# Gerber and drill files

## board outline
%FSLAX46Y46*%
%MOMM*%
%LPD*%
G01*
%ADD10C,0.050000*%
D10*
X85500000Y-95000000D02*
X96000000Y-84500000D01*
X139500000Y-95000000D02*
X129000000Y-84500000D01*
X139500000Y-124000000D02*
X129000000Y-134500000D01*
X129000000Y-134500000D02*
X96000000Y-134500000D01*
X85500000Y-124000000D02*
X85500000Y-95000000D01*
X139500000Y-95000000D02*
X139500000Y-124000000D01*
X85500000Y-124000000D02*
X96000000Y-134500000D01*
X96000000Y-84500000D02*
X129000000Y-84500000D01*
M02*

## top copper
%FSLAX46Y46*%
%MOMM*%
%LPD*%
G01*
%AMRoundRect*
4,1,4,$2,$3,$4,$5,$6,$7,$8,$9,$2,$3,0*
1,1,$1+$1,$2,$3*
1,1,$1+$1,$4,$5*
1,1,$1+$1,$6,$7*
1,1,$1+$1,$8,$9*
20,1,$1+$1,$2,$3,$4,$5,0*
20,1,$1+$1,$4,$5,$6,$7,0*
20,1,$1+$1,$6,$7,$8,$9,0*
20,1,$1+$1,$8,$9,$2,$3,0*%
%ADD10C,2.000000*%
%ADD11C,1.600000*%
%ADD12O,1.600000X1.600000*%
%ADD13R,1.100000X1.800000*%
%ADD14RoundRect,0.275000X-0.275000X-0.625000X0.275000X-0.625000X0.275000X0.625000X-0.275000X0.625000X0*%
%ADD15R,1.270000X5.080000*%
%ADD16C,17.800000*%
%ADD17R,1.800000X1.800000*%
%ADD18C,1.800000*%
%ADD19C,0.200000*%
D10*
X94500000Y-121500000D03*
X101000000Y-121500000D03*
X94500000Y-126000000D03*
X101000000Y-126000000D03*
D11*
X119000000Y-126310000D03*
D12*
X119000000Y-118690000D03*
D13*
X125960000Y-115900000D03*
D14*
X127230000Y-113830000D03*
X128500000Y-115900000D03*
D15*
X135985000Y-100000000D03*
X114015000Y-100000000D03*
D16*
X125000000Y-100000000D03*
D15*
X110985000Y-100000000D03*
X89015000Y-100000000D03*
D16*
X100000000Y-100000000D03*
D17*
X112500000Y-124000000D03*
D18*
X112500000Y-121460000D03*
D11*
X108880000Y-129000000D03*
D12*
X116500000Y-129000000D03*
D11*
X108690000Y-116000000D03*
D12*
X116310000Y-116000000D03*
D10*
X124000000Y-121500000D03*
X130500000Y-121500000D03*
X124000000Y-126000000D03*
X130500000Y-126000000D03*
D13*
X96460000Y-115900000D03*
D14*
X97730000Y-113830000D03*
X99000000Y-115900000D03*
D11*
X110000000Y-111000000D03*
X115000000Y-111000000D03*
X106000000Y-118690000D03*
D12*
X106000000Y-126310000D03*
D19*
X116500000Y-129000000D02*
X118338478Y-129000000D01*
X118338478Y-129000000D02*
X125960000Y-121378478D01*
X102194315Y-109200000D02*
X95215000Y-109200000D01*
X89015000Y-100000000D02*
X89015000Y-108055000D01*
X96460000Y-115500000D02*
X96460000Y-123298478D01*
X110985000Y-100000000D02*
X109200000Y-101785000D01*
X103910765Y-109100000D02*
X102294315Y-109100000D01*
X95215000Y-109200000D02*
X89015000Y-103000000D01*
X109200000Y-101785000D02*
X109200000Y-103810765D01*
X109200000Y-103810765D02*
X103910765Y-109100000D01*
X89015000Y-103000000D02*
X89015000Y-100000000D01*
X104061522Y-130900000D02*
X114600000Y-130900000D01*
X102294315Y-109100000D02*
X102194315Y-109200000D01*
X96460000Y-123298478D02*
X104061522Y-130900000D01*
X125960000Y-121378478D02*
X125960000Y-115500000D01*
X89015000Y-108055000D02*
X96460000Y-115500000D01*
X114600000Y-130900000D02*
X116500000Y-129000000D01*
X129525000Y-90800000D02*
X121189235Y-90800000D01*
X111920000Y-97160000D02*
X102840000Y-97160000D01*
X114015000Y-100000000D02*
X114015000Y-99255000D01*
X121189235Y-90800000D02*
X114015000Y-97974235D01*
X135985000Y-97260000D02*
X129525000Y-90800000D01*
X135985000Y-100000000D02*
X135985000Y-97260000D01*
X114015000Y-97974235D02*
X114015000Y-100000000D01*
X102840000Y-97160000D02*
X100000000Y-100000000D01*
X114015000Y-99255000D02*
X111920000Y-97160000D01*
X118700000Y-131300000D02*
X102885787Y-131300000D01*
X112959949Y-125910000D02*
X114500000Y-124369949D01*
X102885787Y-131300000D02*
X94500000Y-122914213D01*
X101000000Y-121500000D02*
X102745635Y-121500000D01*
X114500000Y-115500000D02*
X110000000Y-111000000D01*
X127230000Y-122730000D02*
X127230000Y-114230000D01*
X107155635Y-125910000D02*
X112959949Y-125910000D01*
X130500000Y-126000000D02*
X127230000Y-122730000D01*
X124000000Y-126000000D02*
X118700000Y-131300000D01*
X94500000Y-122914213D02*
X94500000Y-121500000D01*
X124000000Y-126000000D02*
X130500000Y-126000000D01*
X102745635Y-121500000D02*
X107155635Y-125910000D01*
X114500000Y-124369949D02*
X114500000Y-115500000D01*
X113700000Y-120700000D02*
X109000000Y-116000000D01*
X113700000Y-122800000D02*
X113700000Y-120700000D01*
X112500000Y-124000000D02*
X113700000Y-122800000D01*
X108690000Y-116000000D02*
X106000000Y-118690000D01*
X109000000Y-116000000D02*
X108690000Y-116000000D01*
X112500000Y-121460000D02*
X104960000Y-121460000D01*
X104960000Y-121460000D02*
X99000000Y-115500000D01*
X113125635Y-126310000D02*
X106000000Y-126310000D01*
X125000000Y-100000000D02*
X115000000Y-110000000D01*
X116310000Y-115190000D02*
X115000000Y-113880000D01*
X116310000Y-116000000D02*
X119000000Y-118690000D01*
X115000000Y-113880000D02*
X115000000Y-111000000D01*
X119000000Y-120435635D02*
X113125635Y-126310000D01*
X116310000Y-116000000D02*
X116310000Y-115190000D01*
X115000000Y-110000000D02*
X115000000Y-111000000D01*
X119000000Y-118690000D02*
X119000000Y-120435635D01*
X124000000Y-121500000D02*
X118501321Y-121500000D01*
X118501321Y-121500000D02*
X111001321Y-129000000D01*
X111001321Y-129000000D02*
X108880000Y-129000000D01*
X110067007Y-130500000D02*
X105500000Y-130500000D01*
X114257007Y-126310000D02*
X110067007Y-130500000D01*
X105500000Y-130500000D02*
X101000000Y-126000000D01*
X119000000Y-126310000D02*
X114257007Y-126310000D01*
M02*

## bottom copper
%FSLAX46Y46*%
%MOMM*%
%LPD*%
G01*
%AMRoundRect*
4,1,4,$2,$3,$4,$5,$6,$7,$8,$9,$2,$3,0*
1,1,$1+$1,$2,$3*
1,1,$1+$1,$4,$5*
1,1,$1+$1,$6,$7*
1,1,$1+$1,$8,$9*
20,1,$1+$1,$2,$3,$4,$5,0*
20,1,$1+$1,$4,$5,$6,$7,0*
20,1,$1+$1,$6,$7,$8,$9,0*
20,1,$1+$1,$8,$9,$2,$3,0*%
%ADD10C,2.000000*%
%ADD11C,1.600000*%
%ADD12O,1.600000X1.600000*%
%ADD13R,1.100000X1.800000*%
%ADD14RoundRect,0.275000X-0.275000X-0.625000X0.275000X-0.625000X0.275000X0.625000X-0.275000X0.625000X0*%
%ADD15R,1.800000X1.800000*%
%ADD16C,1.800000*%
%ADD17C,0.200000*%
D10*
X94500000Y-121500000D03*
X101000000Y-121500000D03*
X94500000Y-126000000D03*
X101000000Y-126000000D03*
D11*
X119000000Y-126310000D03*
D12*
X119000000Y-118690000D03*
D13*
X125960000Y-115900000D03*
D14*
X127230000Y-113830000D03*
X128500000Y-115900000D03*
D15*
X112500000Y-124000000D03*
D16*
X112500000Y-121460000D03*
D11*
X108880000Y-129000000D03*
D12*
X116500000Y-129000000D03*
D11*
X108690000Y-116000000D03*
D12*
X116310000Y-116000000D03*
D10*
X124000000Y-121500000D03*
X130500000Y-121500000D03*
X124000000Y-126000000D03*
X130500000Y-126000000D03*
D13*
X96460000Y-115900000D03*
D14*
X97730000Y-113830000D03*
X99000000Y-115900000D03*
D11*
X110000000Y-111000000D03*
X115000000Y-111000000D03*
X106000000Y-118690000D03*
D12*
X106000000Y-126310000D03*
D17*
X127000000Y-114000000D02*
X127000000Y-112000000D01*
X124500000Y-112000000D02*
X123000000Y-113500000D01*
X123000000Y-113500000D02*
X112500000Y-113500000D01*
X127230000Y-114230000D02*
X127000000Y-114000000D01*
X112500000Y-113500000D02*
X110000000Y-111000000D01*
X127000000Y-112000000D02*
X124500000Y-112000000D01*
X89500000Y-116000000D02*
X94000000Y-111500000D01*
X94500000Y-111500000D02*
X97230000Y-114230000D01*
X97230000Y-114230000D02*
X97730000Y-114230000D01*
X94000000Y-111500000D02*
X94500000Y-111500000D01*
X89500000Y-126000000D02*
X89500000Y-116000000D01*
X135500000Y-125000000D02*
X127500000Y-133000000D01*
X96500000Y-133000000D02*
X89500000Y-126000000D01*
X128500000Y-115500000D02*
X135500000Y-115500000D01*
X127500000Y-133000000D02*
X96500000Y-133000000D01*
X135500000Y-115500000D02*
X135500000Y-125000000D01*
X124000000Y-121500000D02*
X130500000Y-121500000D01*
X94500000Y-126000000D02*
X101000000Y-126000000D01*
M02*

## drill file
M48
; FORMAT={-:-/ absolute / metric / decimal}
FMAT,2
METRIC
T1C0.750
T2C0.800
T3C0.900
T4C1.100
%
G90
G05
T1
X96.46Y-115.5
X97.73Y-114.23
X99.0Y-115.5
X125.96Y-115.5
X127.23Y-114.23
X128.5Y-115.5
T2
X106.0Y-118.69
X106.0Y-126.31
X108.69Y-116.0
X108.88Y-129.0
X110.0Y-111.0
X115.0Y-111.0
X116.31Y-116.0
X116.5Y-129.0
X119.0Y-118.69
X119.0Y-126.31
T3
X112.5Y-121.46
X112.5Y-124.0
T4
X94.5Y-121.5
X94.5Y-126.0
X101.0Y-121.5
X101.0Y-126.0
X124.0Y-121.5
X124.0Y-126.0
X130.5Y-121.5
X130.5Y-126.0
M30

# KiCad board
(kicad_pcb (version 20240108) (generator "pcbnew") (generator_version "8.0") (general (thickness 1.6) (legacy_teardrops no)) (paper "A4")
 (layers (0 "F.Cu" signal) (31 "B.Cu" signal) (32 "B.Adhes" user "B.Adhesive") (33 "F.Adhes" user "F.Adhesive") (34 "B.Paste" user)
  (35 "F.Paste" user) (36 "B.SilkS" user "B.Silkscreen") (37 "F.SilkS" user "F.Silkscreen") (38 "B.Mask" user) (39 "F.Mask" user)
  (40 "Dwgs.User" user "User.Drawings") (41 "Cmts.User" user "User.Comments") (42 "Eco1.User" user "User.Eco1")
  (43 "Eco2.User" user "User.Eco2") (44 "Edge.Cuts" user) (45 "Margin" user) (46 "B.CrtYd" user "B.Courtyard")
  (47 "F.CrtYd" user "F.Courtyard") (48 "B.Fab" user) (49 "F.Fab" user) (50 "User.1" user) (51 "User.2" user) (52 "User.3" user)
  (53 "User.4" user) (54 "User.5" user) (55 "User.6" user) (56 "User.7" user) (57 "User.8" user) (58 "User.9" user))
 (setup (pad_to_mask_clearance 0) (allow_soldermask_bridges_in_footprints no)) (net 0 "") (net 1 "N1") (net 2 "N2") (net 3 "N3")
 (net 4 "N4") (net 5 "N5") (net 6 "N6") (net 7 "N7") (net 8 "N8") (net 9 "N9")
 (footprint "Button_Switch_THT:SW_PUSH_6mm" (layer "F.Cu") (at 94.5 121.5)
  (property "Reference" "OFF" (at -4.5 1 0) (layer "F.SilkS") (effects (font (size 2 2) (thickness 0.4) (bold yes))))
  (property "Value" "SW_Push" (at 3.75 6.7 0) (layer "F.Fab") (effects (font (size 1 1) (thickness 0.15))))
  (pad "1" thru_hole circle (at 0 0 90) (size 2 2) (drill 1.1) (layers "*.Cu" "*.Mask") (remove_unused_layers no) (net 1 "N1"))
  (pad "1" thru_hole circle (at 6.5 0 90) (size 2 2) (drill 1.1) (layers "*.Cu" "*.Mask") (remove_unused_layers no) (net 1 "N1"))
  (pad "2" thru_hole circle (at 0 4.5 90) (size 2 2) (drill 1.1) (layers "*.Cu" "*.Mask") (remove_unused_layers no) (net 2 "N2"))
  (pad "2" thru_hole circle (at 6.5 4.5 90) (size 2 2) (drill 1.1) (layers "*.Cu" "*.Mask") (remove_unused_layers no) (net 2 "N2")))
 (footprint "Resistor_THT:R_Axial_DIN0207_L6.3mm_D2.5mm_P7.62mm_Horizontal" (layer "F.Cu") (at 119 126.31 90)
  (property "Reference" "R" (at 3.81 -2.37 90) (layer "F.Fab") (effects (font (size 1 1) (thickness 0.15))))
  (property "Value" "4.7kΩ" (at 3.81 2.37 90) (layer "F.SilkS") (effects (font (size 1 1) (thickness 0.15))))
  (pad "1" thru_hole circle (at 0 0 90) (size 1.6 1.6) (drill 0.8) (layers "*.Cu" "*.Mask") (remove_unused_layers no) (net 2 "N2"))
  (pad "2" thru_hole oval (at 7.62 0 90) (size 1.6 1.6) (drill 0.8) (layers "*.Cu" "*.Mask") (remove_unused_layers no) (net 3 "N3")))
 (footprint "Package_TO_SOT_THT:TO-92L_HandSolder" (layer "F.Cu") (at 125.96 115.5)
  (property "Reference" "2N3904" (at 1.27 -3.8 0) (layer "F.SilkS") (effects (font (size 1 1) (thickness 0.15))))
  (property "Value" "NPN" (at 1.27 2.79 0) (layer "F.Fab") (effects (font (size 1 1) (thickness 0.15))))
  (pad "1" thru_hole rect (at 0 0) (size 1.1 1.8) (drill 0.75 (offset 0 0.4)) (layers "*.Cu" "*.Mask") (remove_unused_layers no)
   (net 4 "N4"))
  (pad "2" thru_hole roundrect (at 1.27 -1.27) (size 1.1 1.8) (drill 0.75 (offset 0 -0.4)) (layers "*.Cu" "*.Mask")
   (remove_unused_layers no) (roundrect_rratio 0.25) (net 1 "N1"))
  (pad "3" thru_hole roundrect (at 2.54 0) (size 1.1 1.8) (drill 0.75 (offset 0 0.4)) (layers "*.Cu" "*.Mask") (remove_unused_layers no)
   (roundrect_rratio 0.25) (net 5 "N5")))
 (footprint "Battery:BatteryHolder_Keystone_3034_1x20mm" (layer "F.Cu") (at 125 100 180)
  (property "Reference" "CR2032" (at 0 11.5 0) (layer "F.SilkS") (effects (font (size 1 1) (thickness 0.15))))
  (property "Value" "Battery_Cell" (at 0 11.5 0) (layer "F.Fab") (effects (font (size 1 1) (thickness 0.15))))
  (pad "1" smd rect (at -10.985 0 180) (size 1.27 5.08) (layers "F.Cu" "F.Paste" "F.Mask") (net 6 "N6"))
  (pad "1" smd rect (at 10.985 0 180) (size 1.27 5.08) (layers "F.Cu" "F.Paste" "F.Mask") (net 6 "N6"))
  (pad "2" smd circle (at 0 0 180) (size 17.8 17.8) (layers "F.Cu" "F.Mask") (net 3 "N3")))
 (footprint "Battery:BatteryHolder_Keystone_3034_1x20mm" (layer "F.Cu") (at 100 100 180)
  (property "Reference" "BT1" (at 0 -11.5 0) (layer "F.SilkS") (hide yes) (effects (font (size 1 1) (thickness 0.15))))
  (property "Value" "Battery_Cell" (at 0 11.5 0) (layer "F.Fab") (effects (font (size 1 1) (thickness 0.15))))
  (pad "1" smd rect (at -10.985 0 180) (size 1.27 5.08) (layers "F.Cu" "F.Paste" "F.Mask") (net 4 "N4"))
  (pad "1" smd rect (at 10.985 0 180) (size 1.27 5.08) (layers "F.Cu" "F.Paste" "F.Mask") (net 4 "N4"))
  (pad "2" smd circle (at 0 0 180) (size 17.8 17.8) (layers "F.Cu" "F.Mask") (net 6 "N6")))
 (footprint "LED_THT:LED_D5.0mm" (layer "F.Cu") (at 112.5 124 90)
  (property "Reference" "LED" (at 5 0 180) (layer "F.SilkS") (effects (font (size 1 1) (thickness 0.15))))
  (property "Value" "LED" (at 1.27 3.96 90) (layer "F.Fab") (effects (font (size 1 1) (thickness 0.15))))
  (pad "1" thru_hole rect (at 0 0 90) (size 1.8 1.8) (drill 0.9) (layers "*.Cu" "*.Mask") (remove_unused_layers no) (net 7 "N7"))
  (pad "2" thru_hole circle (at 2.54 0 90) (size 1.8 1.8) (drill 0.9) (layers "*.Cu" "*.Mask") (remove_unused_layers no) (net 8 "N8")))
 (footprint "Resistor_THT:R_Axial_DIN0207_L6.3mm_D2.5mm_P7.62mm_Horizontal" (layer "F.Cu") (at 108.88 129)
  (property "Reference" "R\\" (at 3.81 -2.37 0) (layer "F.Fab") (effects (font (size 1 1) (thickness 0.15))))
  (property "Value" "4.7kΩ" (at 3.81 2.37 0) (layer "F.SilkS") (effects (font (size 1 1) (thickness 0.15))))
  (pad "1" thru_hole circle (at 0 0) (size 1.6 1.6) (drill 0.8) (layers "*.Cu" "*.Mask") (remove_unused_layers no) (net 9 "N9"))
  (pad "2" thru_hole oval (at 7.62 0) (size 1.6 1.6) (drill 0.8) (layers "*.Cu" "*.Mask") (remove_unused_layers no) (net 4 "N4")))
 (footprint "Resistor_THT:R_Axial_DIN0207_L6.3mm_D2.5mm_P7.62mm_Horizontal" (layer "F.Cu") (at 108.69 116)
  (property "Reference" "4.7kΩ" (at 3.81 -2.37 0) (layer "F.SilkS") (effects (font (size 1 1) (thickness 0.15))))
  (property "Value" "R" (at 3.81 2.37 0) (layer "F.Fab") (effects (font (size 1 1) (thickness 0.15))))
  (pad "1" thru_hole circle (at 0 0) (size 1.6 1.6) (drill 0.8) (layers "*.Cu" "*.Mask") (remove_unused_layers no) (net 7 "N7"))
  (pad "2" thru_hole oval (at 7.62 0) (size 1.6 1.6) (drill 0.8) (layers "*.Cu" "*.Mask") (remove_unused_layers no) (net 3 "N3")))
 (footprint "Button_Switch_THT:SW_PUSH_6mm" (layer "F.Cu") (at 124 121.5)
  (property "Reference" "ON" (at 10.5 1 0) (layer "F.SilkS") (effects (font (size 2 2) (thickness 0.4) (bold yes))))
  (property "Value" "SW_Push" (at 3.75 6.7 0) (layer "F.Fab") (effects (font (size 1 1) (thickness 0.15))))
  (pad "1" thru_hole circle (at 0 0 90) (size 2 2) (drill 1.1) (layers "*.Cu" "*.Mask") (remove_unused_layers no) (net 9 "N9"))
  (pad "1" thru_hole circle (at 6.5 0 90) (size 2 2) (drill 1.1) (layers "*.Cu" "*.Mask") (remove_unused_layers no) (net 9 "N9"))
  (pad "2" thru_hole circle (at 0 4.5 90) (size 2 2) (drill 1.1) (layers "*.Cu" "*.Mask") (remove_unused_layers no) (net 1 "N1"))
  (pad "2" thru_hole circle (at 6.5 4.5 90) (size 2 2) (drill 1.1) (layers "*.Cu" "*.Mask") (remove_unused_layers no) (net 1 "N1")))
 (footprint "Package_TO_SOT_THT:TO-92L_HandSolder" (layer "F.Cu") (at 96.46 115.5)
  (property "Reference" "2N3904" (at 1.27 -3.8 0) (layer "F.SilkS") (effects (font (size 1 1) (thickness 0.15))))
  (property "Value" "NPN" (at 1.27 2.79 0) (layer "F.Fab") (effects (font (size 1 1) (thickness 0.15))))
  (pad "1" thru_hole rect (at 0 0) (size 1.1 1.8) (drill 0.75 (offset 0 0.4)) (layers "*.Cu" "*.Mask") (remove_unused_layers no)
   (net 4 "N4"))
  (pad "2" thru_hole roundrect (at 1.27 -1.27) (size 1.1 1.8) (drill 0.75 (offset 0 -0.4)) (layers "*.Cu" "*.Mask")
   (remove_unused_layers no) (roundrect_rratio 0.25) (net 5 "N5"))
  (pad "3" thru_hole roundrect (at 2.54 0) (size 1.1 1.8) (drill 0.75 (offset 0 0.4)) (layers "*.Cu" "*.Mask") (remove_unused_layers no)
   (roundrect_rratio 0.25) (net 8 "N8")))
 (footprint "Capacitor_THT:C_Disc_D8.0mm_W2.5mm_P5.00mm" (layer "F.Cu") (at 110 111)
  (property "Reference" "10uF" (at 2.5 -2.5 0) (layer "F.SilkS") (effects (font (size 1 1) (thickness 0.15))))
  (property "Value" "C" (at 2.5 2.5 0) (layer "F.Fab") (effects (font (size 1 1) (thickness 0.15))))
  (pad "1" thru_hole circle (at 0 0) (size 1.6 1.6) (drill 0.8) (layers "*.Cu" "*.Mask") (remove_unused_layers no) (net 1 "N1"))
  (pad "2" thru_hole circle (at 5 0) (size 1.6 1.6) (drill 0.8) (layers "*.Cu" "*.Mask") (remove_unused_layers no) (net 3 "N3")))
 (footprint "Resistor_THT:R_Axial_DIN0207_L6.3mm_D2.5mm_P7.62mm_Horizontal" (layer "F.Cu") (at 106 118.69 -90)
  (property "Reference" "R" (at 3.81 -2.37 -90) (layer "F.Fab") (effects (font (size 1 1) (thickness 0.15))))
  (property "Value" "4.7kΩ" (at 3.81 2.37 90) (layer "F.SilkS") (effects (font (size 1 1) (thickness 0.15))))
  (pad "1" thru_hole circle (at 0 0 270) (size 1.6 1.6) (drill 0.8) (layers "*.Cu" "*.Mask") (remove_unused_layers no) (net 7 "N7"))
  (pad "2" thru_hole oval (at 7.62 0 270) (size 1.6 1.6) (drill 0.8) (layers "*.Cu" "*.Mask") (remove_unused_layers no) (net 3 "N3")))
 (gr_line (start 85.5 95) (end 96 84.5) (stroke (width 0.05) (type default)) (layer "Edge.Cuts"))
 (gr_line (start 139.5 95) (end 129 84.5) (stroke (width 0.05) (type default)) (layer "Edge.Cuts"))
 (gr_line (start 139.5 124) (end 129 134.5) (stroke (width 0.05) (type default)) (layer "Edge.Cuts"))
 (gr_line (start 129 134.5) (end 96 134.5) (stroke (width 0.05) (type default)) (layer "Edge.Cuts"))
 (gr_line (start 85.5 124) (end 85.5 95) (stroke (width 0.05) (type default)) (layer "Edge.Cuts"))
 (gr_line (start 139.5 95) (end 139.5 124) (stroke (width 0.05) (type default)) (layer "Edge.Cuts"))
 (gr_line (start 85.5 124) (end 96 134.5) (stroke (width 0.05) (type default)) (layer "Edge.Cuts"))
 (gr_line (start 96 84.5) (end 129 84.5) (stroke (width 0.05) (type default)) (layer "Edge.Cuts"))
 (segment (start 116.5 129) (end 118.338478 129) (width 0.2) (layer "F.Cu") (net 4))
 (segment (start 118.338478 129) (end 125.96 121.378478) (width 0.2) (layer "F.Cu") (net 4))
 (segment (start 102.194315 109.2) (end 95.215 109.2) (width 0.2) (layer "F.Cu") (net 4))
 (segment (start 89.015 100) (end 89.015 108.055) (width 0.2) (layer "F.Cu") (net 4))
 (segment (start 96.46 115.5) (end 96.46 123.298478) (width 0.2) (layer "F.Cu") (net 4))
 (segment (start 110.985 100) (end 109.2 101.785) (width 0.2) (layer "F.Cu") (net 4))
 (segment (start 103.910765 109.1) (end 102.294315 109.1) (width 0.2) (layer "F.Cu") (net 4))
 (segment (start 95.215 109.2) (end 89.015 103) (width 0.2) (layer "F.Cu") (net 4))
 (segment (start 109.2 101.785) (end 109.2 103.810765) (width 0.2) (layer "F.Cu") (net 4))
 (segment (start 109.2 103.810765) (end 103.910765 109.1) (width 0.2) (layer "F.Cu") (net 4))
 (segment (start 89.015 103) (end 89.015 100) (width 0.2) (layer "F.Cu") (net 4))
 (segment (start 104.061522 130.9) (end 114.6 130.9) (width 0.2) (layer "F.Cu") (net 4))
 (segment (start 102.294315 109.1) (end 102.194315 109.2) (width 0.2) (layer "F.Cu") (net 4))
 (segment (start 96.46 123.298478) (end 104.061522 130.9) (width 0.2) (layer "F.Cu") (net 4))
 (segment (start 125.96 121.378478) (end 125.96 115.5) (width 0.2) (layer "F.Cu") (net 4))
 (segment (start 89.015 108.055) (end 96.46 115.5) (width 0.2) (layer "F.Cu") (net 4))
 (segment (start 114.6 130.9) (end 116.5 129) (width 0.2) (layer "F.Cu") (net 4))
 (segment (start 129.525 90.8) (end 121.189235 90.8) (width 0.2) (layer "F.Cu") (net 6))
 (segment (start 111.92 97.16) (end 102.84 97.16) (width 0.2) (layer "F.Cu") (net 6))
 (segment (start 114.015 100) (end 114.015 99.255) (width 0.2) (layer "F.Cu") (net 6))
 (segment (start 121.189235 90.8) (end 114.015 97.974235) (width 0.2) (layer "F.Cu") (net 6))
 (segment (start 135.985 97.26) (end 129.525 90.8) (width 0.2) (layer "F.Cu") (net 6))
 (segment (start 135.985 100) (end 135.985 97.26) (width 0.2) (layer "F.Cu") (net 6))
 (segment (start 114.015 97.974235) (end 114.015 100) (width 0.2) (layer "F.Cu") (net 6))
 (segment (start 102.84 97.16) (end 100 100) (width 0.2) (layer "F.Cu") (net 6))
 (segment (start 114.015 99.255) (end 111.92 97.16) (width 0.2) (layer "F.Cu") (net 6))
 (segment (start 118.7 131.3) (end 102.885787 131.3) (width 0.2) (layer "F.Cu") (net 1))
 (segment (start 112.959949 125.91) (end 114.5 124.369949) (width 0.2) (layer "F.Cu") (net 1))
 (segment (start 102.885787 131.3) (end 94.5 122.914213) (width 0.2) (layer "F.Cu") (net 1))
 (segment (start 101 121.5) (end 102.745635 121.5) (width 0.2) (layer "F.Cu") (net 1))
 (segment (start 114.5 115.5) (end 110 111) (width 0.2) (layer "F.Cu") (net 1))
 (segment (start 127.23 122.73) (end 127.23 114.23) (width 0.2) (layer "F.Cu") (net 1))
 (segment (start 107.155635 125.91) (end 112.959949 125.91) (width 0.2) (layer "F.Cu") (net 1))
 (segment (start 130.5 126) (end 127.23 122.73) (width 0.2) (layer "F.Cu") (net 1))
 (segment (start 124 126) (end 118.7 131.3) (width 0.2) (layer "F.Cu") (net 1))
 (segment (start 94.5 122.914213) (end 94.5 121.5) (width 0.2) (layer "F.Cu") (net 1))
 (segment (start 124 126) (end 130.5 126) (width 0.2) (layer "F.Cu") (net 1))
 (segment (start 102.745635 121.5) (end 107.155635 125.91) (width 0.2) (layer "F.Cu") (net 1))
 (segment (start 114.5 124.369949) (end 114.5 115.5) (width 0.2) (layer "F.Cu") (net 1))
 (segment (start 127 114) (end 127 112) (width 0.2) (layer "B.Cu") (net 1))
 (segment (start 124.5 112) (end 123 113.5) (width 0.2) (layer "B.Cu") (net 1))
 (segment (start 123 113.5) (end 112.5 113.5) (width 0.2) (layer "B.Cu") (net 1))
 (segment (start 127.23 114.23) (end 127 114) (width 0.2) (layer "B.Cu") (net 1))
 (segment (start 112.5 113.5) (end 110 111) (width 0.2) (layer "B.Cu") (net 1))
 (segment (start 127 112) (end 124.5 112) (width 0.2) (layer "B.Cu") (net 1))
 (segment (start 113.7 120.7) (end 109 116) (width 0.2) (layer "F.Cu") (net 7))
 (segment (start 113.7 122.8) (end 113.7 120.7) (width 0.2) (layer "F.Cu") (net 7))
 (segment (start 112.5 124) (end 113.7 122.8) (width 0.2) (layer "F.Cu") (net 7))
 (segment (start 108.69 116) (end 106 118.69) (width 0.2) (layer "F.Cu") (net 7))
 (segment (start 109 116) (end 108.69 116) (width 0.2) (layer "F.Cu") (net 7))
 (segment (start 112.5 121.46) (end 104.96 121.46) (width 0.2) (layer "F.Cu") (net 8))
 (segment (start 104.96 121.46) (end 99 115.5) (width 0.2) (layer "F.Cu") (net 8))
 (segment (start 89.5 116) (end 94 111.5) (width 0.2) (layer "B.Cu") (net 5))
 (segment (start 94.5 111.5) (end 97.23 114.23) (width 0.2) (layer "B.Cu") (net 5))
 (segment (start 97.23 114.23) (end 97.73 114.23) (width 0.2) (layer "B.Cu") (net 5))
 (segment (start 94 111.5) (end 94.5 111.5) (width 0.2) (layer "B.Cu") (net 5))
 (segment (start 89.5 126) (end 89.5 116) (width 0.2) (layer "B.Cu") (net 5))
 (segment (start 135.5 125) (end 127.5 133) (width 0.2) (layer "B.Cu") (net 5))
 (segment (start 96.5 133) (end 89.5 126) (width 0.2) (layer "B.Cu") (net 5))
 (segment (start 128.5 115.5) (end 135.5 115.5) (width 0.2) (layer "B.Cu") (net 5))
 (segment (start 127.5 133) (end 96.5 133) (width 0.2) (layer "B.Cu") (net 5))
 (segment (start 135.5 115.5) (end 135.5 125) (width 0.2) (layer "B.Cu") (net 5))
 (segment (start 113.125635 126.31) (end 106 126.31) (width 0.2) (layer "F.Cu") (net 3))
 (segment (start 125 100) (end 115 110) (width 0.2) (layer "F.Cu") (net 3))
 (segment (start 116.31 115.19) (end 115 113.88) (width 0.2) (layer "F.Cu") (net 3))
 (segment (start 116.31 116) (end 119 118.69) (width 0.2) (layer "F.Cu") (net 3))
 (segment (start 115 113.88) (end 115 111) (width 0.2) (layer "F.Cu") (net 3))
 (segment (start 119 120.435635) (end 113.125635 126.31) (width 0.2) (layer "F.Cu") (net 3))
 (segment (start 116.31 116) (end 116.31 115.19) (width 0.2) (layer "F.Cu") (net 3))
 (segment (start 115 110) (end 115 111) (width 0.2) (layer "F.Cu") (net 3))
 (segment (start 119 118.69) (end 119 120.435635) (width 0.2) (layer "F.Cu") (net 3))
 (segment (start 124 121.5) (end 118.501321 121.5) (width 0.2) (layer "F.Cu") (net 9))
 (segment (start 118.501321 121.5) (end 111.001321 129) (width 0.2) (layer "F.Cu") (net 9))
 (segment (start 111.001321 129) (end 108.88 129) (width 0.2) (layer "F.Cu") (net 9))
 (segment (start 124 121.5) (end 130.5 121.5) (width 0.2) (layer "B.Cu") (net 9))
 (segment (start 110.067007 130.5) (end 105.5 130.5) (width 0.2) (layer "F.Cu") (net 2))
 (segment (start 114.257007 126.31) (end 110.067007 130.5) (width 0.2) (layer "F.Cu") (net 2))
 (segment (start 105.5 130.5) (end 101 126) (width 0.2) (layer "F.Cu") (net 2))
 (segment (start 119 126.31) (end 114.257007 126.31) (width 0.2) (layer "F.Cu") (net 2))
 (segment (start 94.5 126) (end 101 126) (width 0.2) (layer "B.Cu") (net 2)))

